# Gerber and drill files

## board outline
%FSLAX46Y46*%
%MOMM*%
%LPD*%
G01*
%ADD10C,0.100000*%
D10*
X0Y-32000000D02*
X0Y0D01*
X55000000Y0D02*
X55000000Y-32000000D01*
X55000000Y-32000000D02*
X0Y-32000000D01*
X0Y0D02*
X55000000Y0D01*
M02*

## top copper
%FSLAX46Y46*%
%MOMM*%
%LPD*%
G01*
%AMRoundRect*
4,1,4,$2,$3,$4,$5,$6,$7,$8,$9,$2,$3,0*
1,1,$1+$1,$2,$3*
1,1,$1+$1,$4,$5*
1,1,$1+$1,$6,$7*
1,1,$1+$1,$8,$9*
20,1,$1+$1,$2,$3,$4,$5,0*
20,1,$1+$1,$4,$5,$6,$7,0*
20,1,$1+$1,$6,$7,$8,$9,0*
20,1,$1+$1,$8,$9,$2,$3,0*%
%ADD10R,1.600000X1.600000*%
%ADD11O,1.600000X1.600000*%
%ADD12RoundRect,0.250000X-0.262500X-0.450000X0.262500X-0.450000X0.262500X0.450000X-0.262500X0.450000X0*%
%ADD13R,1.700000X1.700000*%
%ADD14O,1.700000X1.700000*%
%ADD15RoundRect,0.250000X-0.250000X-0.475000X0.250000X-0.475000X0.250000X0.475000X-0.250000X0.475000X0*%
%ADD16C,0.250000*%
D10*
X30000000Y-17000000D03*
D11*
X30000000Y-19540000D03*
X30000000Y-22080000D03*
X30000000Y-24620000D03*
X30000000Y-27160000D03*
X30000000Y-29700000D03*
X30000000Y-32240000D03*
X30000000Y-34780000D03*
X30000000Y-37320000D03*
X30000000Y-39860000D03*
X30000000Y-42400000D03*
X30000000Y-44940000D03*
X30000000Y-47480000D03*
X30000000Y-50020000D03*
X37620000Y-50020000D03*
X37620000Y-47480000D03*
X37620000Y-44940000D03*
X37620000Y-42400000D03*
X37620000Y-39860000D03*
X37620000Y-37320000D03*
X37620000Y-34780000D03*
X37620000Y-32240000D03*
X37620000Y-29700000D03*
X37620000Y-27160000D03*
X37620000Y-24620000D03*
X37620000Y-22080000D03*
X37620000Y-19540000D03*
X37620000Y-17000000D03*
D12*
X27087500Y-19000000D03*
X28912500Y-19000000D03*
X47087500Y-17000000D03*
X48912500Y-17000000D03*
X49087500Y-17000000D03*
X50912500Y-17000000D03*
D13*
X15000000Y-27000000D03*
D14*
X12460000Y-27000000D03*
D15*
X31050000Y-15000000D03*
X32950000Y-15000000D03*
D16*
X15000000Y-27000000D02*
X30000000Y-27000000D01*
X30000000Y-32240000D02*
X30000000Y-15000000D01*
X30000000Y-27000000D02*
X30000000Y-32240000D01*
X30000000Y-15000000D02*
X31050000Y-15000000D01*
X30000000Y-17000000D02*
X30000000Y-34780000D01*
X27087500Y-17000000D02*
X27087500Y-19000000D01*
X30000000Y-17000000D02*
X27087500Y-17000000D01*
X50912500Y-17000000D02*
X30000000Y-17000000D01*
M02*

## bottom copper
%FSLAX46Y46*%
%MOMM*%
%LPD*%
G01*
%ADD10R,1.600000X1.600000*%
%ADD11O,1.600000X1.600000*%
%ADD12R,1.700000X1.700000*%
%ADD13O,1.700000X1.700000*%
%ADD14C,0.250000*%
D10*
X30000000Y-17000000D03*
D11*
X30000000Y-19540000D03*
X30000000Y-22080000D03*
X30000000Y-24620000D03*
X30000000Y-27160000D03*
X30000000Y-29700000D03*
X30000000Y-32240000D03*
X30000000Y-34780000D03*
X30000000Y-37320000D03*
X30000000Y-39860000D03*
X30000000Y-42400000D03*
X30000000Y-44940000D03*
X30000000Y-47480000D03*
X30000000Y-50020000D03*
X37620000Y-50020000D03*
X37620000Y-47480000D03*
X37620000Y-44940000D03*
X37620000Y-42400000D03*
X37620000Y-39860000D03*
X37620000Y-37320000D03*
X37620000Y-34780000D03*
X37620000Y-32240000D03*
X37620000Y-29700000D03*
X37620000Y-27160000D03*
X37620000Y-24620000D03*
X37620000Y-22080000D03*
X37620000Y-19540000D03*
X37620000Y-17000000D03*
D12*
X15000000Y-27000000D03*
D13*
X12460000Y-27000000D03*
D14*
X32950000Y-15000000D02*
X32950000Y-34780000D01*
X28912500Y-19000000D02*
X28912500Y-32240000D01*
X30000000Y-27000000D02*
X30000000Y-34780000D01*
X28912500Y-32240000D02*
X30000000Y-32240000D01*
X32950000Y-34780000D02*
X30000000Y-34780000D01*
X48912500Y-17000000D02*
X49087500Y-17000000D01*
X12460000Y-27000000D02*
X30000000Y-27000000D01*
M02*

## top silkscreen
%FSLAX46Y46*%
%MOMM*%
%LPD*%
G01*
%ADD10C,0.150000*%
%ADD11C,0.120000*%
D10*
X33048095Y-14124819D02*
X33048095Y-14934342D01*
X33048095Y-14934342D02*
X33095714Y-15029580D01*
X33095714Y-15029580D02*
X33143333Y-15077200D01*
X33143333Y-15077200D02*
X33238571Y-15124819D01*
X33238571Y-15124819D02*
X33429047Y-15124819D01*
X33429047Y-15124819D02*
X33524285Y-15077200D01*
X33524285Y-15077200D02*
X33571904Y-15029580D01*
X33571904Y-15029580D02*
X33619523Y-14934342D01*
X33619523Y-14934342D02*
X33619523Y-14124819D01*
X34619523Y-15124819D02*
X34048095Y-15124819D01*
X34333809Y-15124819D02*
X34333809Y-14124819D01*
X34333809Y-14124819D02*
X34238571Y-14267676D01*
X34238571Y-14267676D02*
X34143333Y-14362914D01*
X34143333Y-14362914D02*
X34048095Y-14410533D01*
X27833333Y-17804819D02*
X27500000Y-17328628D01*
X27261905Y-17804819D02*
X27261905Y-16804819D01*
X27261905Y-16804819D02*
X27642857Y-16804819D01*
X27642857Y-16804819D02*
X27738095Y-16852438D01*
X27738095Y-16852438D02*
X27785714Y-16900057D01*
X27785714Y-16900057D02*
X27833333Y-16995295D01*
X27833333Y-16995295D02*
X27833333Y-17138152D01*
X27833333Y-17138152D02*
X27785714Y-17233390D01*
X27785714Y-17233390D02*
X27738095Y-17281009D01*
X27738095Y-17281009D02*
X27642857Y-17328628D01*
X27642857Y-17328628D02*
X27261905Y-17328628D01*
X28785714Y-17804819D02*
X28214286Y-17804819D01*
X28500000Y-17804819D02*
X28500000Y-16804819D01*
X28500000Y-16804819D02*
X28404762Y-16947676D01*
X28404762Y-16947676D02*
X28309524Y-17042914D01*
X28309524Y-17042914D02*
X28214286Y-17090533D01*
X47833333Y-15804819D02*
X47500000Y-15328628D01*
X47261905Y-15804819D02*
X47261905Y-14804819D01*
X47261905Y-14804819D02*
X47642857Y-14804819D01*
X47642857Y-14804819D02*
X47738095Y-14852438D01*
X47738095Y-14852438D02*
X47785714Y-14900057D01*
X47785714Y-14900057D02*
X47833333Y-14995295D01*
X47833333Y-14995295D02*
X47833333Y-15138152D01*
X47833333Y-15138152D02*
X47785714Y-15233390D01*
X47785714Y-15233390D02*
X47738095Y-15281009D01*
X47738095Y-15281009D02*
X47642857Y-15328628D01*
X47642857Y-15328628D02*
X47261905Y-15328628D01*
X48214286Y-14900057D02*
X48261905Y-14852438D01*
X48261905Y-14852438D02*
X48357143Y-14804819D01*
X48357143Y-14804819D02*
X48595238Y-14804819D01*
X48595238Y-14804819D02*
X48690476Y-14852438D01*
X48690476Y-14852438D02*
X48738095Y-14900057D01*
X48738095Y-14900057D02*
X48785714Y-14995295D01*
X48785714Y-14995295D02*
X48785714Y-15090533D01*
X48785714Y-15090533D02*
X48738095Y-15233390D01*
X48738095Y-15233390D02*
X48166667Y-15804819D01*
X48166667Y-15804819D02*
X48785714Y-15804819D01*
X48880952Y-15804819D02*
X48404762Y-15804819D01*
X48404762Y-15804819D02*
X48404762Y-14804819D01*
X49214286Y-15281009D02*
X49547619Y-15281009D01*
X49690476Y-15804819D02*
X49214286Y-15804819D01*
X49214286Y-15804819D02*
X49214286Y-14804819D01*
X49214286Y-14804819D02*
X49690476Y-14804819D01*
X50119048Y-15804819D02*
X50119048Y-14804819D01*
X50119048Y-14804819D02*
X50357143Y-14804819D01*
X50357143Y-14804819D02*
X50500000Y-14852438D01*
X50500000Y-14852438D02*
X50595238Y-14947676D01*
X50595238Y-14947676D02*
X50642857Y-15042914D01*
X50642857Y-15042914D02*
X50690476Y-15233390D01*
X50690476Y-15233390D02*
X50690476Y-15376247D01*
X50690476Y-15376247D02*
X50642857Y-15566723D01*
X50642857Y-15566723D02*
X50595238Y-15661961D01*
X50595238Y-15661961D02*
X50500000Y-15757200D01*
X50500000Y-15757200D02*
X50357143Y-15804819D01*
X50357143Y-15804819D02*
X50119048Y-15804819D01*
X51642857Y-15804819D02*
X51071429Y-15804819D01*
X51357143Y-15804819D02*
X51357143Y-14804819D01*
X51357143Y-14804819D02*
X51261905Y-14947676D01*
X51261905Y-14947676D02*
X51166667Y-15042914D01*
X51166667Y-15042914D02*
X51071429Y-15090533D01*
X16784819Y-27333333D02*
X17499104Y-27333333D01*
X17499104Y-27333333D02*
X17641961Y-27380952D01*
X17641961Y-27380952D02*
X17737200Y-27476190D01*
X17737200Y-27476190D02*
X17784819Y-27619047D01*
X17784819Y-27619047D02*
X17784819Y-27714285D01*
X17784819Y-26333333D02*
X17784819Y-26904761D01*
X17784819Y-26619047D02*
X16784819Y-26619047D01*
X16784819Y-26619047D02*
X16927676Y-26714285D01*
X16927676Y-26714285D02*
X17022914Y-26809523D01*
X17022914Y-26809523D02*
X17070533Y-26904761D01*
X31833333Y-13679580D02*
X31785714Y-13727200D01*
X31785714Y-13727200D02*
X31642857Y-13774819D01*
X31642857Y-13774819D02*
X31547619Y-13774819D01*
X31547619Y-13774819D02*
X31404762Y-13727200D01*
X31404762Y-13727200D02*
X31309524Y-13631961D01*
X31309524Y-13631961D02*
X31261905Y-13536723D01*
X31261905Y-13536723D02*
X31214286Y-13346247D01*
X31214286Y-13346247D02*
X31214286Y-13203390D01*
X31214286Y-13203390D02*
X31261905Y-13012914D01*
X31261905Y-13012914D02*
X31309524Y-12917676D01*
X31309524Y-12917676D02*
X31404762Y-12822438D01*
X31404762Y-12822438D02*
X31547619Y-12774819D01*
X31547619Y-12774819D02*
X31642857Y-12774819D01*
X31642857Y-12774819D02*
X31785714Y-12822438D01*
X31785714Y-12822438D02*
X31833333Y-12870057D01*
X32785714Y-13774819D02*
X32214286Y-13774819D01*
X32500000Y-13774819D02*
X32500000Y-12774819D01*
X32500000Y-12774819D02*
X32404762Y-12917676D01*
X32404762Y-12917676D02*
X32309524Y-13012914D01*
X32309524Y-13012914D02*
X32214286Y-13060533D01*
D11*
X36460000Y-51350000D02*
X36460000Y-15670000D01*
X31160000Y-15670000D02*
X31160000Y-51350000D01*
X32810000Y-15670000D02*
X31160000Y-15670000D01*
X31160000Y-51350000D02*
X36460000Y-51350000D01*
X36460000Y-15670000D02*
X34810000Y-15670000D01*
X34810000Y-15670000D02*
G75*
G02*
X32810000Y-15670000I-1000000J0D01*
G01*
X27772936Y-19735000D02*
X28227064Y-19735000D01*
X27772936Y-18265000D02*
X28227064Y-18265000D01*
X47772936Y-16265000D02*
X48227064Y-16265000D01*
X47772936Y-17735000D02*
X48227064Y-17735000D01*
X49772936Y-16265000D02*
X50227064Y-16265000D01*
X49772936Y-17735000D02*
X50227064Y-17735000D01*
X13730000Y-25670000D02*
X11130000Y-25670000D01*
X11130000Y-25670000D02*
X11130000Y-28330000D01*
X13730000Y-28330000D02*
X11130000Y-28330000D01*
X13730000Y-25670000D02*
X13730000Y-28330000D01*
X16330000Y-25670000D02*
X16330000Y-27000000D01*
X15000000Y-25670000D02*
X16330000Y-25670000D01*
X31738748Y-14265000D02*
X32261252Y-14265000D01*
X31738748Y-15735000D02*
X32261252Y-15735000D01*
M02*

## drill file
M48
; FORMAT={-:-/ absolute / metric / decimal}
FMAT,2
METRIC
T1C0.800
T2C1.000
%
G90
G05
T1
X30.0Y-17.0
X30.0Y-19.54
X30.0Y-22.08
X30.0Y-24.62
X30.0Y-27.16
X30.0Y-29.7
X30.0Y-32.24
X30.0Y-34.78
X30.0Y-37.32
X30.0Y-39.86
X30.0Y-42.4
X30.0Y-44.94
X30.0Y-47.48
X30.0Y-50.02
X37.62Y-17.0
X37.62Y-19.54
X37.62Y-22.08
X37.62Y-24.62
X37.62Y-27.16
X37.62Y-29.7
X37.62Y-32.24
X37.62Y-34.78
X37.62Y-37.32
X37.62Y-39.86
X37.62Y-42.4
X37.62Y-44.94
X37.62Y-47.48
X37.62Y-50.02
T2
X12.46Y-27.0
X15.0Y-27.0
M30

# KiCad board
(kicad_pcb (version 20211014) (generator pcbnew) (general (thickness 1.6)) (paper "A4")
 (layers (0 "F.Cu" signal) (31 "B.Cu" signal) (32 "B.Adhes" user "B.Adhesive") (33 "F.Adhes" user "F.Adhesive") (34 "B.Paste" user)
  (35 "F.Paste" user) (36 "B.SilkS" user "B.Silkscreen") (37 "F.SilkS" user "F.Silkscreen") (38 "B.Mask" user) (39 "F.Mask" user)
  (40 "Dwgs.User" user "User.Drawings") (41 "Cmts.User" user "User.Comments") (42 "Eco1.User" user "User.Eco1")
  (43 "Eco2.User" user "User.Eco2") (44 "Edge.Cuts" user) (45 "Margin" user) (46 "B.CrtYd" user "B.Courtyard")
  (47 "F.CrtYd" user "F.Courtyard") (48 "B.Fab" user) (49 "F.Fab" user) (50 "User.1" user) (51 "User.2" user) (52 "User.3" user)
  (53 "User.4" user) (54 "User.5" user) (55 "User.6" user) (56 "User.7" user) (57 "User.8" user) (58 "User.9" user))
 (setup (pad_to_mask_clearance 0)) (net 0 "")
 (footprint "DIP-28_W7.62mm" (layer "F.Cu") (at 30 17)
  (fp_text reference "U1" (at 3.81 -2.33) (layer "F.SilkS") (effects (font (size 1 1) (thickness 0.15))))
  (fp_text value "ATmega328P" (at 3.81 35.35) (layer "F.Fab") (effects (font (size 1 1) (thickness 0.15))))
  (fp_line (start 6.46 34.35) (end 6.46 -1.33) (layer "F.SilkS") (width 0.12))
  (fp_line (start 1.16 -1.33) (end 1.16 34.35) (layer "F.SilkS") (width 0.12))
  (fp_line (start 2.81 -1.33) (end 1.16 -1.33) (layer "F.SilkS") (width 0.12))
  (fp_line (start 1.16 34.35) (end 6.46 34.35) (layer "F.SilkS") (width 0.12))
  (fp_line (start 6.46 -1.33) (end 4.81 -1.33) (layer "F.SilkS") (width 0.12))
  (fp_arc (start 4.81 -1.33) (mid 3.81 -0.33) (end 2.81 -1.33) (layer "F.SilkS") (width 0.12))
  (pad "1" thru_hole rect (at 0 0) (size 1.6 1.6) (drill 0.8) (layers *.Cu *.Mask))
  (pad "2" thru_hole oval (at 0 2.54) (size 1.6 1.6) (drill 0.8) (layers *.Cu *.Mask))
  (pad "3" thru_hole oval (at 0 5.08) (size 1.6 1.6) (drill 0.8) (layers *.Cu *.Mask))
  (pad "4" thru_hole oval (at 0 7.62) (size 1.6 1.6) (drill 0.8) (layers *.Cu *.Mask))
  (pad "5" thru_hole oval (at 0 10.16) (size 1.6 1.6) (drill 0.8) (layers *.Cu *.Mask))
  (pad "6" thru_hole oval (at 0 12.7) (size 1.6 1.6) (drill 0.8) (layers *.Cu *.Mask))
  (pad "7" thru_hole oval (at 0 15.24) (size 1.6 1.6) (drill 0.8) (layers *.Cu *.Mask))
  (pad "8" thru_hole oval (at 0 17.78) (size 1.6 1.6) (drill 0.8) (layers *.Cu *.Mask))
  (pad "9" thru_hole oval (at 0 20.32) (size 1.6 1.6) (drill 0.8) (layers *.Cu *.Mask))
  (pad "10" thru_hole oval (at 0 22.86) (size 1.6 1.6) (drill 0.8) (layers *.Cu *.Mask))
  (pad "11" thru_hole oval (at 0 25.4) (size 1.6 1.6) (drill 0.8) (layers *.Cu *.Mask))
  (pad "12" thru_hole oval (at 0 27.94) (size 1.6 1.6) (drill 0.8) (layers *.Cu *.Mask))
  (pad "13" thru_hole oval (at 0 30.48) (size 1.6 1.6) (drill 0.8) (layers *.Cu *.Mask))
  (pad "14" thru_hole oval (at 0 33.02) (size 1.6 1.6) (drill 0.8) (layers *.Cu *.Mask))
  (pad "15" thru_hole oval (at 7.62 33.02) (size 1.6 1.6) (drill 0.8) (layers *.Cu *.Mask))
  (pad "16" thru_hole oval (at 7.62 30.48) (size 1.6 1.6) (drill 0.8) (layers *.Cu *.Mask))
  (pad "17" thru_hole oval (at 7.62 27.94) (size 1.6 1.6) (drill 0.8) (layers *.Cu *.Mask))
  (pad "18" thru_hole oval (at 7.62 25.4) (size 1.6 1.6) (drill 0.8) (layers *.Cu *.Mask))
  (pad "19" thru_hole oval (at 7.62 22.86) (size 1.6 1.6) (drill 0.8) (layers *.Cu *.Mask))
  (pad "20" thru_hole oval (at 7.62 20.32) (size 1.6 1.6) (drill 0.8) (layers *.Cu *.Mask))
  (pad "21" thru_hole oval (at 7.62 17.78) (size 1.6 1.6) (drill 0.8) (layers *.Cu *.Mask))
  (pad "22" thru_hole oval (at 7.62 15.24) (size 1.6 1.6) (drill 0.8) (layers *.Cu *.Mask))
  (pad "23" thru_hole oval (at 7.62 12.7) (size 1.6 1.6) (drill 0.8) (layers *.Cu *.Mask))
  (pad "24" thru_hole oval (at 7.62 10.16) (size 1.6 1.6) (drill 0.8) (layers *.Cu *.Mask))
  (pad "25" thru_hole oval (at 7.62 7.62) (size 1.6 1.6) (drill 0.8) (layers *.Cu *.Mask))
  (pad "26" thru_hole oval (at 7.62 5.08) (size 1.6 1.6) (drill 0.8) (layers *.Cu *.Mask))
  (pad "27" thru_hole oval (at 7.62 2.54) (size 1.6 1.6) (drill 0.8) (layers *.Cu *.Mask))
  (pad "28" thru_hole oval (at 7.62 0) (size 1.6 1.6) (drill 0.8) (layers *.Cu *.Mask)))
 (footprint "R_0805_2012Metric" (layer "F.Cu") (at 28 19)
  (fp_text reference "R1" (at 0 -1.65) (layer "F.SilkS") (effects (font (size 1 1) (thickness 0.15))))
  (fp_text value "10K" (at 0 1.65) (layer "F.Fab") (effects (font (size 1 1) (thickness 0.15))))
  (fp_line (start -0.227064 0.735) (end 0.227064 0.735) (layer "F.SilkS") (width 0.12))
  (fp_line (start -0.227064 -0.735) (end 0.227064 -0.735) (layer "F.SilkS") (width 0.12))
  (pad "1" smd roundrect (at -0.9125 0) (size 1.025 1.4) (layers "F.Cu" "F.Paste" "F.Mask") (roundrect_rratio 0.243902))
  (pad "2" smd roundrect (at 0.9125 0) (size 1.025 1.4) (layers "F.Cu" "F.Paste" "F.Mask") (roundrect_rratio 0.243902)))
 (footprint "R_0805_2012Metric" (layer "F.Cu") (at 48 17)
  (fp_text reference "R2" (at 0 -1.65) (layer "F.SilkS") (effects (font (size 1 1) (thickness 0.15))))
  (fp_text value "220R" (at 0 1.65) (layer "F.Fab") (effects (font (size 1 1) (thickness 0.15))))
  (fp_line (start -0.227064 -0.735) (end 0.227064 -0.735) (layer "F.SilkS") (width 0.12))
  (fp_line (start -0.227064 0.735) (end 0.227064 0.735) (layer "F.SilkS") (width 0.12))
  (pad "1" smd roundrect (at -0.9125 0) (size 1.025 1.4) (layers "F.Cu" "F.Paste" "F.Mask") (roundrect_rratio 0.243902))
  (pad "2" smd roundrect (at 0.9125 0) (size 1.025 1.4) (layers "F.Cu" "F.Paste" "F.Mask") (roundrect_rratio 0.243902)))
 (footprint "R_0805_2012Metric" (layer "F.Cu") (at 50 17)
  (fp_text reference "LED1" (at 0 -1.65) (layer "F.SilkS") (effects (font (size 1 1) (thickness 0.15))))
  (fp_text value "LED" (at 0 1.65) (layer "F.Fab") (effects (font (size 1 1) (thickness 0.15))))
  (fp_line (start -0.227064 -0.735) (end 0.227064 -0.735) (layer "F.SilkS") (width 0.12))
  (fp_line (start -0.227064 0.735) (end 0.227064 0.735) (layer "F.SilkS") (width 0.12))
  (pad "1" smd roundrect (at -0.9125 0) (size 1.025 1.4) (layers "F.Cu" "F.Paste" "F.Mask") (roundrect_rratio 0.243902))
  (pad "2" smd roundrect (at 0.9125 0) (size 1.025 1.4) (layers "F.Cu" "F.Paste" "F.Mask") (roundrect_rratio 0.243902)))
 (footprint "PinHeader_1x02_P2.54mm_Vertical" (layer "F.Cu") (at 15 27 -90)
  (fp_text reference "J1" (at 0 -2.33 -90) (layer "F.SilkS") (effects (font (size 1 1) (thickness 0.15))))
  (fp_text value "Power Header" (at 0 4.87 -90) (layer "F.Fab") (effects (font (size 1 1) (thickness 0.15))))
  (fp_line (start -1.33 1.27) (end -1.33 3.87) (layer "F.SilkS") (width 0.12))
  (fp_line (start -1.33 3.87) (end 1.33 3.87) (layer "F.SilkS") (width 0.12))
  (fp_line (start 1.33 1.27) (end 1.33 3.87) (layer "F.SilkS") (width 0.12))
  (fp_line (start -1.33 1.27) (end 1.33 1.27) (layer "F.SilkS") (width 0.12))
  (fp_line (start -1.33 -1.33) (end 0 -1.33) (layer "F.SilkS") (width 0.12))
  (fp_line (start -1.33 0) (end -1.33 -1.33) (layer "F.SilkS") (width 0.12))
  (pad "1" thru_hole rect (at 0 0 270) (size 1.7 1.7) (drill 1) (layers *.Cu *.Mask))
  (pad "2" thru_hole oval (at 0 2.54 270) (size 1.7 1.7) (drill 1) (layers *.Cu *.Mask)))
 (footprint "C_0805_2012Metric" (layer "F.Cu") (at 32 15)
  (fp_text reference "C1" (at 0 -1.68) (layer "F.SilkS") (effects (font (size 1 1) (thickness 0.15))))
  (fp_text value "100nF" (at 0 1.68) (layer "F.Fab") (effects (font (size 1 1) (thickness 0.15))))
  (fp_line (start -0.261252 -0.735) (end 0.261252 -0.735) (layer "F.SilkS") (width 0.12))
  (fp_line (start -0.261252 0.735) (end 0.261252 0.735) (layer "F.SilkS") (width 0.12))
  (pad "1" smd roundrect (at -0.95 0) (size 1 1.45) (layers "F.Cu" "F.Paste" "F.Mask") (roundrect_rratio 0.25))
  (pad "2" smd roundrect (at 0.95 0) (size 1 1.45) (layers "F.Cu" "F.Paste" "F.Mask") (roundrect_rratio 0.25)))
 (gr_line (start 0 32) (end 0 0) (layer "Edge.Cuts") (width 0.1))
 (gr_line (start 55 0) (end 55 32) (layer "Edge.Cuts") (width 0.1))
 (gr_line (start 55 32) (end 0 32) (layer "Edge.Cuts") (width 0.1))
 (gr_line (start 0 0) (end 55 0) (layer "Edge.Cuts") (width 0.1))
 (segment (start 15 27) (end 30 27) (width 0.25) (layer "F.Cu") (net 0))
 (segment (start 30 32.24) (end 30 15) (width 0.25) (layer "F.Cu") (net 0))
 (segment (start 30 27) (end 30 32.24) (width 0.25) (layer "F.Cu") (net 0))
 (segment (start 30 15) (end 31.05 15) (width 0.25) (layer "F.Cu") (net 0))
 (segment (start 30 17) (end 30 34.78) (width 0.25) (layer "F.Cu") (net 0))
 (segment (start 27.0875 17) (end 27.0875 19) (width 0.25) (layer "F.Cu") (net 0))
 (segment (start 30 17) (end 27.0875 17) (width 0.25) (layer "F.Cu") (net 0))
 (segment (start 50.9125 17) (end 30 17) (width 0.25) (layer "F.Cu") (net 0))
 (segment (start 32.95 15) (end 32.95 34.78) (width 0.25) (layer "B.Cu") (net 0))
 (segment (start 28.9125 19) (end 28.9125 32.24) (width 0.25) (layer "B.Cu") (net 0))
 (segment (start 30 27) (end 30 34.78) (width 0.25) (layer "B.Cu") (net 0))
 (segment (start 28.9125 32.24) (end 30 32.24) (width 0.25) (layer "B.Cu") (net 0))
 (segment (start 32.95 34.78) (end 30 34.78) (width 0.25) (layer "B.Cu") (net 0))
 (segment (start 48.9125 17) (end 49.0875 17) (width 0.25) (layer "B.Cu") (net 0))
 (segment (start 12.46 27) (end 30 27) (width 0.25) (layer "B.Cu") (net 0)))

